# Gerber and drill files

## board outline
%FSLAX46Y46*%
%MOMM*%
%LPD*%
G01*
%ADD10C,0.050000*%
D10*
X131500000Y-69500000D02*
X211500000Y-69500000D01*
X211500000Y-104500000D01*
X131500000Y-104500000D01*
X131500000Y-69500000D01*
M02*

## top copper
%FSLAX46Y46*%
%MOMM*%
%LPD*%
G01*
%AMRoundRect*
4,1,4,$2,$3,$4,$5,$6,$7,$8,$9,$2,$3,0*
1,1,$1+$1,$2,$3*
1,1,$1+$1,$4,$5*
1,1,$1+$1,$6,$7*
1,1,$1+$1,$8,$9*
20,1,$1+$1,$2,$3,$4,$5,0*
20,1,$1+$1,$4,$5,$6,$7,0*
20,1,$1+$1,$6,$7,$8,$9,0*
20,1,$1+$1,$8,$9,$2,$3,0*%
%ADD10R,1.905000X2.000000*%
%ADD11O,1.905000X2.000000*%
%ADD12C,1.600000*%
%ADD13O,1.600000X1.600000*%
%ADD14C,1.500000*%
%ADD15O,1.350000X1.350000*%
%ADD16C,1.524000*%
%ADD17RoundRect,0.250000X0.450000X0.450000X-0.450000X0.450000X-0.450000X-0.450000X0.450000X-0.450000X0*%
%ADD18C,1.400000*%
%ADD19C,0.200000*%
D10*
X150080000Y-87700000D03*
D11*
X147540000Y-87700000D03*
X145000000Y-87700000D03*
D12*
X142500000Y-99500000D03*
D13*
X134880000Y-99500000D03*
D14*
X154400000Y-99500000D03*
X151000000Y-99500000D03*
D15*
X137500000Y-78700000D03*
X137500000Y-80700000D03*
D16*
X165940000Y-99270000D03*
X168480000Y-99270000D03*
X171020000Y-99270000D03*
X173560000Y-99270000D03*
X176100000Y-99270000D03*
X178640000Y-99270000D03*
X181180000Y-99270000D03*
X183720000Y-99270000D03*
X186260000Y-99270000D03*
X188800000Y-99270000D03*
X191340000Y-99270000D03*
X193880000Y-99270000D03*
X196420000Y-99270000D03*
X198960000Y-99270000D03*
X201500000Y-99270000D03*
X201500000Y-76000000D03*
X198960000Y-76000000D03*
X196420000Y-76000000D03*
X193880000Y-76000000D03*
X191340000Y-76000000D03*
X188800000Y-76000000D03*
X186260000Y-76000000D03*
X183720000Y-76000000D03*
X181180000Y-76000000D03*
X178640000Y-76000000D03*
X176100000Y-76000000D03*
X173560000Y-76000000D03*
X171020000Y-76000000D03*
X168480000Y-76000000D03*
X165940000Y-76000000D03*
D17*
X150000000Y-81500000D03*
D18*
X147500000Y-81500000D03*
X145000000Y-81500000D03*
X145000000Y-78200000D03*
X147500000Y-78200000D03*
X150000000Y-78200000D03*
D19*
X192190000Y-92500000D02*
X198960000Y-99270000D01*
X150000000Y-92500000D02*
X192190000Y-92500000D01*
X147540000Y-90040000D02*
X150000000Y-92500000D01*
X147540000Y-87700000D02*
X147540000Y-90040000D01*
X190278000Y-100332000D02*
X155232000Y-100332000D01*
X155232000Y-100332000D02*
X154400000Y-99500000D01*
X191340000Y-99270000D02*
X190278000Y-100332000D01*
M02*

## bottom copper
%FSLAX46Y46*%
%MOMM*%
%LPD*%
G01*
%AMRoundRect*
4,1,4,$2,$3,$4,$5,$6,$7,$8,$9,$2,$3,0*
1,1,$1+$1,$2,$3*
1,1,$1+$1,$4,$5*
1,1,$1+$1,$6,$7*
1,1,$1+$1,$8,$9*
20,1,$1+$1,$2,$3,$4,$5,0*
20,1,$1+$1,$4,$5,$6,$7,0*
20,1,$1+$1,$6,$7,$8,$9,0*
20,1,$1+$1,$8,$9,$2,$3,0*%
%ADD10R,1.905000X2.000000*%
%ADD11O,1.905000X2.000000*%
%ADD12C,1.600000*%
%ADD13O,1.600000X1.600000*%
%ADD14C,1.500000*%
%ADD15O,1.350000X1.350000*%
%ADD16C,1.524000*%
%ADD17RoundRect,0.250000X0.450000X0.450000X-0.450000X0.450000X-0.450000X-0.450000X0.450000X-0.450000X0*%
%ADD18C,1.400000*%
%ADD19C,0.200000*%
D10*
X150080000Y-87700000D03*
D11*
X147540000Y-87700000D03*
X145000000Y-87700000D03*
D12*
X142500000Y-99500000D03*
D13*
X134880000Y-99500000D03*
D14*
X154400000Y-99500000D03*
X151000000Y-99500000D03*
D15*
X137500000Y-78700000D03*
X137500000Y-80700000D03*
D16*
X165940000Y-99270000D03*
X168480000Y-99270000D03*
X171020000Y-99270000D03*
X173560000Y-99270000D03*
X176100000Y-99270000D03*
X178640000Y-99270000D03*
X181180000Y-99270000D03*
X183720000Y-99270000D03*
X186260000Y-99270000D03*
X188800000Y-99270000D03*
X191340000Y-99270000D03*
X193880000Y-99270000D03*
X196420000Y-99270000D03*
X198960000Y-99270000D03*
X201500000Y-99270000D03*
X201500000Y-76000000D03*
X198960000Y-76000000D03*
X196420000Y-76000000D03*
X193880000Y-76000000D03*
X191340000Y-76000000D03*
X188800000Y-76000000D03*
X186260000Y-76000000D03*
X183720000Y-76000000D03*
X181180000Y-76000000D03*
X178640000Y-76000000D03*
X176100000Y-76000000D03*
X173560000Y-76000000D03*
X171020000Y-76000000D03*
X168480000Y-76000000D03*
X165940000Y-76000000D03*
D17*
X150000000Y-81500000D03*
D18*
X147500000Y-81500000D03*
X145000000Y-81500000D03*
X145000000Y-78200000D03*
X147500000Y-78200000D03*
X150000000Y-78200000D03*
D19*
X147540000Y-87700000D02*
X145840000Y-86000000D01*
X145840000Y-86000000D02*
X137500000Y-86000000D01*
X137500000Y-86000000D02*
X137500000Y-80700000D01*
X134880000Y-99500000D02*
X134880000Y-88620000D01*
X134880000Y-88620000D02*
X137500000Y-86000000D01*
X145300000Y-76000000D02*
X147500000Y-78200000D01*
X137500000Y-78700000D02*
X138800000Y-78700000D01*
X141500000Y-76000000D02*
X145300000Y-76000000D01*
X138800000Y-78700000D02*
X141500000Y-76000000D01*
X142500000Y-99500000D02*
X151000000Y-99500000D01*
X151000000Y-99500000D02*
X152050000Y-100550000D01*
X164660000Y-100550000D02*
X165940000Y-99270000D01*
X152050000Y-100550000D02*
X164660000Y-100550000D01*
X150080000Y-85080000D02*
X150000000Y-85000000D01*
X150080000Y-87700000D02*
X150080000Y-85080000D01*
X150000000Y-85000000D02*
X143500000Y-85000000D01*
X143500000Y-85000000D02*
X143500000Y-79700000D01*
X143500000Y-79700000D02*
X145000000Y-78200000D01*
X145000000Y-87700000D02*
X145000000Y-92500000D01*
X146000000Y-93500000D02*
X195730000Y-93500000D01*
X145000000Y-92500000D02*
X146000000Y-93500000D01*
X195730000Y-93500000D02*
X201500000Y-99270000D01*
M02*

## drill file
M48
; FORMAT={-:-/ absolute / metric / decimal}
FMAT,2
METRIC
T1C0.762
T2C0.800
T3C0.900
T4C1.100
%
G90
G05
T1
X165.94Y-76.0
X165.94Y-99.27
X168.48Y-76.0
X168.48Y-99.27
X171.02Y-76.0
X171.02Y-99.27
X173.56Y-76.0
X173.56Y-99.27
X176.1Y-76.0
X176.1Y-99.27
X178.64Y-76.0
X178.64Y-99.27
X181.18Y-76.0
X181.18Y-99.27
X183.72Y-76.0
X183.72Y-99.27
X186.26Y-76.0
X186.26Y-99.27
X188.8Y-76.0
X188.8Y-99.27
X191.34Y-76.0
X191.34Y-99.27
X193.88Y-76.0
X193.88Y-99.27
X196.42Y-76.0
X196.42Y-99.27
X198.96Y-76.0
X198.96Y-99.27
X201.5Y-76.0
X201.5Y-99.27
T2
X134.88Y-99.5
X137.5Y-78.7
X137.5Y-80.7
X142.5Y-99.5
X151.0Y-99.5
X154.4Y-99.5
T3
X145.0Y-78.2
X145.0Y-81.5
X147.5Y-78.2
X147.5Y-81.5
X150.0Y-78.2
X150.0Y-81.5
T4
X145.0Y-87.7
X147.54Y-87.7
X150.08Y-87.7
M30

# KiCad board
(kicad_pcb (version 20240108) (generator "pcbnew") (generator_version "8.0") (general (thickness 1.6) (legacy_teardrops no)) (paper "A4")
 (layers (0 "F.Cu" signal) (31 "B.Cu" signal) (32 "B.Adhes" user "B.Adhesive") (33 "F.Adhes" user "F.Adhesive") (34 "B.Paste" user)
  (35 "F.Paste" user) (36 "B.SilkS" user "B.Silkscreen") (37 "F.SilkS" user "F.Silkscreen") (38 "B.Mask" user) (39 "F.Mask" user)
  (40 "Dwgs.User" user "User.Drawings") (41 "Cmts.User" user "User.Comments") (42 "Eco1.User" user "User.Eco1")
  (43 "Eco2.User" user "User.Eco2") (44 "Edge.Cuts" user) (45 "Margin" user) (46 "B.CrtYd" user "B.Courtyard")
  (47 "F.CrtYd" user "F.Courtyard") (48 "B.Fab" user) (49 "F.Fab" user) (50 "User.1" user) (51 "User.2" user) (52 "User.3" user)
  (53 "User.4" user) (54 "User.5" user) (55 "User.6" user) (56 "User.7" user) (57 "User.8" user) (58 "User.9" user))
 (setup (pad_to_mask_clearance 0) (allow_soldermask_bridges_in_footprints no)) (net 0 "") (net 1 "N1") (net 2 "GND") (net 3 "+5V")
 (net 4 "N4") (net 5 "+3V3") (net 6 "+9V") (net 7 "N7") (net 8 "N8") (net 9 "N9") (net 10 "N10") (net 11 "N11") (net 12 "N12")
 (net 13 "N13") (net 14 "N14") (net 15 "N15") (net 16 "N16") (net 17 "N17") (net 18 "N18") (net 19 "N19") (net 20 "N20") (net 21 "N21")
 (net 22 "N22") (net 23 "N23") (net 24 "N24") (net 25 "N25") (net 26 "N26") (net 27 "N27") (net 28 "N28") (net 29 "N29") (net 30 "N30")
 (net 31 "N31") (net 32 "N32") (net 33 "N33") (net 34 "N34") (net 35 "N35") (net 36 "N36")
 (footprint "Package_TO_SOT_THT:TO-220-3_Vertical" (layer "F.Cu") (at 150.08 87.7 180)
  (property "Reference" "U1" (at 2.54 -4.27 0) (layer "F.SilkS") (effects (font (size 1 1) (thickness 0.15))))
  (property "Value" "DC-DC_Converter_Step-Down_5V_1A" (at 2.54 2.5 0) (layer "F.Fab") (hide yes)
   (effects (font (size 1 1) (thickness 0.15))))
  (pad "1" thru_hole rect (at 0 0 180) (size 1.905 2) (drill 1.1) (layers "*.Cu" "*.Mask") (remove_unused_layers no) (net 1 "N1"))
  (pad "2" thru_hole oval (at 2.54 0 180) (size 1.905 2) (drill 1.1) (layers "*.Cu" "*.Mask") (remove_unused_layers no) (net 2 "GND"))
  (pad "3" thru_hole oval (at 5.08 0 180) (size 1.905 2) (drill 1.1) (layers "*.Cu" "*.Mask") (remove_unused_layers no) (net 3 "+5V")))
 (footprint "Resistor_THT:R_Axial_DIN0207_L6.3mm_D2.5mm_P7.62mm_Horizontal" (layer "F.Cu") (at 142.5 99.5 180)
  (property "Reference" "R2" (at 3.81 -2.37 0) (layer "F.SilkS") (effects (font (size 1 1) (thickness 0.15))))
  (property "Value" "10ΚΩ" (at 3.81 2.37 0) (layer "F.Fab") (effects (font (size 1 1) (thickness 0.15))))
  (pad "1" thru_hole circle (at 0 0 180) (size 1.6 1.6) (drill 0.8) (layers "*.Cu" "*.Mask") (remove_unused_layers no) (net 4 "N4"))
  (pad "2" thru_hole oval (at 7.62 0 180) (size 1.6 1.6) (drill 0.8) (layers "*.Cu" "*.Mask") (remove_unused_layers no) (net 2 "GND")))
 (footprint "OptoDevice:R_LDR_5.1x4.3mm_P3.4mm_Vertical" (layer "F.Cu") (at 154.4 99.5 180)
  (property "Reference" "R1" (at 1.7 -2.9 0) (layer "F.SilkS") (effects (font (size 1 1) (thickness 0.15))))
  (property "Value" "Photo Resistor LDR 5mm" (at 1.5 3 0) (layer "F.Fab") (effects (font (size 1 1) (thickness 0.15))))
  (pad "1" thru_hole circle (at 0 0 180) (size 1.5 1.5) (drill 0.8) (layers "*.Cu" "*.Mask") (remove_unused_layers no) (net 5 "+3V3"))
  (pad "2" thru_hole circle (at 3.4 0 180) (size 1.5 1.5) (drill 0.8) (layers "*.Cu" "*.Mask") (remove_unused_layers no) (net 4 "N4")))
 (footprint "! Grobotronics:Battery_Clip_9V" (layer "F.Cu") (at 137.5 79.2)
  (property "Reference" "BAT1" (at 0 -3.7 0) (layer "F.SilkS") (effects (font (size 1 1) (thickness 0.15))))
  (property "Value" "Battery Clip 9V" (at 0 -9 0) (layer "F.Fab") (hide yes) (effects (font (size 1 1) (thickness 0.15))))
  (pad "+" thru_hole oval (at 0 -0.5) (size 1.35 1.35) (drill 0.8) (layers "*.Cu" "*.Mask") (remove_unused_layers no) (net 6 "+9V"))
  (pad "-" thru_hole oval (at 0 1.5) (size 1.35 1.35) (drill 0.8) (layers "*.Cu" "*.Mask") (remove_unused_layers no) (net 2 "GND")))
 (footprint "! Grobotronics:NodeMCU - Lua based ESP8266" (layer "F.Cu") (at 183.72 87.77 90)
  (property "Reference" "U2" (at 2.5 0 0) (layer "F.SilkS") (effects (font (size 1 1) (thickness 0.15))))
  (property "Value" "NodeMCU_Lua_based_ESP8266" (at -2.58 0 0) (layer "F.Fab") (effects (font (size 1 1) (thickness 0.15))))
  (pad "1" thru_hole circle (at -11.5 -17.78 90) (size 1.524 1.524) (drill 0.762) (layers "*.Cu" "*.Mask") (remove_unused_layers no)
   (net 4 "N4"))
  (pad "2" thru_hole circle (at -11.5 -15.24 90) (size 1.524 1.524) (drill 0.762) (layers "*.Cu" "*.Mask") (remove_unused_layers no)
   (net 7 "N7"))
  (pad "3" thru_hole circle (at -11.5 -12.7 90) (size 1.524 1.524) (drill 0.762) (layers "*.Cu" "*.Mask") (remove_unused_layers no)
   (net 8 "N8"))
  (pad "4" thru_hole circle (at -11.5 -10.16 90) (size 1.524 1.524) (drill 0.762) (layers "*.Cu" "*.Mask") (remove_unused_layers no)
   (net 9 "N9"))
  (pad "5" thru_hole circle (at -11.5 -7.62 90) (size 1.524 1.524) (drill 0.762) (layers "*.Cu" "*.Mask") (remove_unused_layers no)
   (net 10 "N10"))
  (pad "6" thru_hole circle (at -11.5 -5.08 90) (size 1.524 1.524) (drill 0.762) (layers "*.Cu" "*.Mask") (remove_unused_layers no)
   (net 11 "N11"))
  (pad "7" thru_hole circle (at -11.5 -2.54 90) (size 1.524 1.524) (drill 0.762) (layers "*.Cu" "*.Mask") (remove_unused_layers no)
   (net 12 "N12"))
  (pad "8" thru_hole circle (at -11.5 0 90) (size 1.524 1.524) (drill 0.762) (layers "*.Cu" "*.Mask") (remove_unused_layers no)
   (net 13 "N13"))
  (pad "9" thru_hole circle (at -11.5 2.54 90) (size 1.524 1.524) (drill 0.762) (layers "*.Cu" "*.Mask") (remove_unused_layers no)
   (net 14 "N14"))
  (pad "10" thru_hole circle (at -11.5 5.08 90) (size 1.524 1.524) (drill 0.762) (layers "*.Cu" "*.Mask") (remove_unused_layers no)
   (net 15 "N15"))
  (pad "11" thru_hole circle (at -11.5 7.62 90) (size 1.524 1.524) (drill 0.762) (layers "*.Cu" "*.Mask") (remove_unused_layers no)
   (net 5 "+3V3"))
  (pad "12" thru_hole circle (at -11.5 10.16 90) (size 1.524 1.524) (drill 0.762) (layers "*.Cu" "*.Mask") (remove_unused_layers no)
   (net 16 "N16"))
  (pad "13" thru_hole circle (at -11.5 12.7 90) (size 1.524 1.524) (drill 0.762) (layers "*.Cu" "*.Mask") (remove_unused_layers no)
   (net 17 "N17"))
  (pad "14" thru_hole circle (at -11.5 15.24 90) (size 1.524 1.524) (drill 0.762) (layers "*.Cu" "*.Mask") (remove_unused_layers no)
   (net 2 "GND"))
  (pad "15" thru_hole circle (at -11.5 17.78 90) (size 1.524 1.524) (drill 0.762) (layers "*.Cu" "*.Mask") (remove_unused_layers no)
   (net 3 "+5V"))
  (pad "16" thru_hole circle (at 11.77 17.78 90) (size 1.524 1.524) (drill 0.762) (layers "*.Cu" "*.Mask") (remove_unused_layers no)
   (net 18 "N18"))
  (pad "17" thru_hole circle (at 11.77 15.24 90) (size 1.524 1.524) (drill 0.762) (layers "*.Cu" "*.Mask") (remove_unused_layers no)
   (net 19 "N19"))
  (pad "18" thru_hole circle (at 11.77 12.7 90) (size 1.524 1.524) (drill 0.762) (layers "*.Cu" "*.Mask") (remove_unused_layers no)
   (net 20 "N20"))
  (pad "19" thru_hole circle (at 11.77 10.16 90) (size 1.524 1.524) (drill 0.762) (layers "*.Cu" "*.Mask") (remove_unused_layers no)
   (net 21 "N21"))
  (pad "20" thru_hole circle (at 11.77 7.62 90) (size 1.524 1.524) (drill 0.762) (layers "*.Cu" "*.Mask") (remove_unused_layers no)
   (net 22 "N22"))
  (pad "21" thru_hole circle (at 11.77 5.08 90) (size 1.524 1.524) (drill 0.762) (layers "*.Cu" "*.Mask") (remove_unused_layers no)
   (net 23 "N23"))
  (pad "22" thru_hole circle (at 11.77 2.54 90) (size 1.524 1.524) (drill 0.762) (layers "*.Cu" "*.Mask") (remove_unused_layers no)
   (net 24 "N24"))
  (pad "23" thru_hole circle (at 11.77 0 90) (size 1.524 1.524) (drill 0.762) (layers "*.Cu" "*.Mask") (remove_unused_layers no)
   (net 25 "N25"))
  (pad "24" thru_hole circle (at 11.77 -2.54 90) (size 1.524 1.524) (drill 0.762) (layers "*.Cu" "*.Mask") (remove_unused_layers no)
   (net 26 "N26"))
  (pad "25" thru_hole circle (at 11.77 -5.08 90) (size 1.524 1.524) (drill 0.762) (layers "*.Cu" "*.Mask") (remove_unused_layers no)
   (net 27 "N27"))
  (pad "26" thru_hole circle (at 11.77 -7.62 90) (size 1.524 1.524) (drill 0.762) (layers "*.Cu" "*.Mask") (remove_unused_layers no)
   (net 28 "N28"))
  (pad "27" thru_hole circle (at 11.77 -10.16 90) (size 1.524 1.524) (drill 0.762) (layers "*.Cu" "*.Mask") (remove_unused_layers no)
   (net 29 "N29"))
  (pad "28" thru_hole circle (at 11.77 -12.7 90) (size 1.524 1.524) (drill 0.762) (layers "*.Cu" "*.Mask") (remove_unused_layers no)
   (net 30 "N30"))
  (pad "29" thru_hole circle (at 11.77 -15.24 90) (size 1.524 1.524) (drill 0.762) (layers "*.Cu" "*.Mask") (remove_unused_layers no)
   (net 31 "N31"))
  (pad "30" thru_hole circle (at 11.77 -17.78 90) (size 1.524 1.524) (drill 0.762) (layers "*.Cu" "*.Mask") (remove_unused_layers no)
   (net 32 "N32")))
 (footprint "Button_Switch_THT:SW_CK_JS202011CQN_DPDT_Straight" (layer "F.Cu") (at 150 81.5 180)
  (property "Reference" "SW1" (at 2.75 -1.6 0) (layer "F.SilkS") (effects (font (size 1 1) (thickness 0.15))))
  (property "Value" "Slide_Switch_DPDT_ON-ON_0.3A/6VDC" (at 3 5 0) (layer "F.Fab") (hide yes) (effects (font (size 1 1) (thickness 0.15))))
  (pad "1" thru_hole roundrect (at 0 0 180) (size 1.4 1.4) (drill 0.9) (layers "*.Cu" "*.Mask") (remove_unused_layers no)
   (roundrect_rratio 0.1785714286) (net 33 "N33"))
  (pad "2" thru_hole circle (at 2.5 0 180) (size 1.4 1.4) (drill 0.9) (layers "*.Cu" "*.Mask") (remove_unused_layers no) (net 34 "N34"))
  (pad "3" thru_hole circle (at 5 0 180) (size 1.4 1.4) (drill 0.9) (layers "*.Cu" "*.Mask") (remove_unused_layers no) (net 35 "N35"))
  (pad "4" thru_hole circle (at 5 3.3 180) (size 1.4 1.4) (drill 0.9) (layers "*.Cu" "*.Mask") (remove_unused_layers no) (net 1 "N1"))
  (pad "5" thru_hole circle (at 2.5 3.3 180) (size 1.4 1.4) (drill 0.9) (layers "*.Cu" "*.Mask") (remove_unused_layers no) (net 6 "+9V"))
  (pad "6" thru_hole circle (at 0 3.3 180) (size 1.4 1.4) (drill 0.9) (layers "*.Cu" "*.Mask") (remove_unused_layers no) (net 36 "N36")))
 (gr_rect (start 131.5 69.5) (end 211.5 104.5) (stroke (width 0.05) (type default)) (fill none) (layer "Edge.Cuts"))
 (segment (start 192.19 92.5) (end 198.96 99.27) (width 0.2) (layer "F.Cu") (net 2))
 (segment (start 150 92.5) (end 192.19 92.5) (width 0.2) (layer "F.Cu") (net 2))
 (segment (start 147.54 90.04) (end 150 92.5) (width 0.2) (layer "F.Cu") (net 2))
 (segment (start 147.54 87.7) (end 147.54 90.04) (width 0.2) (layer "F.Cu") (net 2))
 (segment (start 147.54 87.7) (end 145.84 86) (width 0.2) (layer "B.Cu") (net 2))
 (segment (start 145.84 86) (end 137.5 86) (width 0.2) (layer "B.Cu") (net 2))
 (segment (start 137.5 86) (end 137.5 80.7) (width 0.2) (layer "B.Cu") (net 2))
 (segment (start 134.88 99.5) (end 134.88 88.62) (width 0.2) (layer "B.Cu") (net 2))
 (segment (start 134.88 88.62) (end 137.5 86) (width 0.2) (layer "B.Cu") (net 2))
 (segment (start 145.3 76) (end 147.5 78.2) (width 0.2) (layer "B.Cu") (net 6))
 (segment (start 137.5 78.7) (end 138.8 78.7) (width 0.2) (layer "B.Cu") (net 6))
 (segment (start 141.5 76) (end 145.3 76) (width 0.2) (layer "B.Cu") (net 6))
 (segment (start 138.8 78.7) (end 141.5 76) (width 0.2) (layer "B.Cu") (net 6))
 (segment (start 190.278 100.332) (end 155.232 100.332) (width 0.2) (layer "F.Cu") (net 5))
 (segment (start 155.232 100.332) (end 154.4 99.5) (width 0.2) (layer "F.Cu") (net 5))
 (segment (start 191.34 99.27) (end 190.278 100.332) (width 0.2) (layer "F.Cu") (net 5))
 (segment (start 142.5 99.5) (end 151 99.5) (width 0.2) (layer "B.Cu") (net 4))
 (segment (start 151 99.5) (end 152.05 100.55) (width 0.2) (layer "B.Cu") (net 4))
 (segment (start 164.66 100.55) (end 165.94 99.27) (width 0.2) (layer "B.Cu") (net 4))
 (segment (start 152.05 100.55) (end 164.66 100.55) (width 0.2) (layer "B.Cu") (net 4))
 (segment (start 150.08 85.08) (end 150 85) (width 0.2) (layer "B.Cu") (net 1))
 (segment (start 150.08 87.7) (end 150.08 85.08) (width 0.2) (layer "B.Cu") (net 1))
 (segment (start 150 85) (end 143.5 85) (width 0.2) (layer "B.Cu") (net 1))
 (segment (start 143.5 85) (end 143.5 79.7) (width 0.2) (layer "B.Cu") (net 1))
 (segment (start 143.5 79.7) (end 145 78.2) (width 0.2) (layer "B.Cu") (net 1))
 (segment (start 145 87.7) (end 145 92.5) (width 0.2) (layer "B.Cu") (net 3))
 (segment (start 146 93.5) (end 195.73 93.5) (width 0.2) (layer "B.Cu") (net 3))
 (segment (start 145 92.5) (end 146 93.5) (width 0.2) (layer "B.Cu") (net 3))
 (segment (start 195.73 93.5) (end 201.5 99.27) (width 0.2) (layer "B.Cu") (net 3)))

